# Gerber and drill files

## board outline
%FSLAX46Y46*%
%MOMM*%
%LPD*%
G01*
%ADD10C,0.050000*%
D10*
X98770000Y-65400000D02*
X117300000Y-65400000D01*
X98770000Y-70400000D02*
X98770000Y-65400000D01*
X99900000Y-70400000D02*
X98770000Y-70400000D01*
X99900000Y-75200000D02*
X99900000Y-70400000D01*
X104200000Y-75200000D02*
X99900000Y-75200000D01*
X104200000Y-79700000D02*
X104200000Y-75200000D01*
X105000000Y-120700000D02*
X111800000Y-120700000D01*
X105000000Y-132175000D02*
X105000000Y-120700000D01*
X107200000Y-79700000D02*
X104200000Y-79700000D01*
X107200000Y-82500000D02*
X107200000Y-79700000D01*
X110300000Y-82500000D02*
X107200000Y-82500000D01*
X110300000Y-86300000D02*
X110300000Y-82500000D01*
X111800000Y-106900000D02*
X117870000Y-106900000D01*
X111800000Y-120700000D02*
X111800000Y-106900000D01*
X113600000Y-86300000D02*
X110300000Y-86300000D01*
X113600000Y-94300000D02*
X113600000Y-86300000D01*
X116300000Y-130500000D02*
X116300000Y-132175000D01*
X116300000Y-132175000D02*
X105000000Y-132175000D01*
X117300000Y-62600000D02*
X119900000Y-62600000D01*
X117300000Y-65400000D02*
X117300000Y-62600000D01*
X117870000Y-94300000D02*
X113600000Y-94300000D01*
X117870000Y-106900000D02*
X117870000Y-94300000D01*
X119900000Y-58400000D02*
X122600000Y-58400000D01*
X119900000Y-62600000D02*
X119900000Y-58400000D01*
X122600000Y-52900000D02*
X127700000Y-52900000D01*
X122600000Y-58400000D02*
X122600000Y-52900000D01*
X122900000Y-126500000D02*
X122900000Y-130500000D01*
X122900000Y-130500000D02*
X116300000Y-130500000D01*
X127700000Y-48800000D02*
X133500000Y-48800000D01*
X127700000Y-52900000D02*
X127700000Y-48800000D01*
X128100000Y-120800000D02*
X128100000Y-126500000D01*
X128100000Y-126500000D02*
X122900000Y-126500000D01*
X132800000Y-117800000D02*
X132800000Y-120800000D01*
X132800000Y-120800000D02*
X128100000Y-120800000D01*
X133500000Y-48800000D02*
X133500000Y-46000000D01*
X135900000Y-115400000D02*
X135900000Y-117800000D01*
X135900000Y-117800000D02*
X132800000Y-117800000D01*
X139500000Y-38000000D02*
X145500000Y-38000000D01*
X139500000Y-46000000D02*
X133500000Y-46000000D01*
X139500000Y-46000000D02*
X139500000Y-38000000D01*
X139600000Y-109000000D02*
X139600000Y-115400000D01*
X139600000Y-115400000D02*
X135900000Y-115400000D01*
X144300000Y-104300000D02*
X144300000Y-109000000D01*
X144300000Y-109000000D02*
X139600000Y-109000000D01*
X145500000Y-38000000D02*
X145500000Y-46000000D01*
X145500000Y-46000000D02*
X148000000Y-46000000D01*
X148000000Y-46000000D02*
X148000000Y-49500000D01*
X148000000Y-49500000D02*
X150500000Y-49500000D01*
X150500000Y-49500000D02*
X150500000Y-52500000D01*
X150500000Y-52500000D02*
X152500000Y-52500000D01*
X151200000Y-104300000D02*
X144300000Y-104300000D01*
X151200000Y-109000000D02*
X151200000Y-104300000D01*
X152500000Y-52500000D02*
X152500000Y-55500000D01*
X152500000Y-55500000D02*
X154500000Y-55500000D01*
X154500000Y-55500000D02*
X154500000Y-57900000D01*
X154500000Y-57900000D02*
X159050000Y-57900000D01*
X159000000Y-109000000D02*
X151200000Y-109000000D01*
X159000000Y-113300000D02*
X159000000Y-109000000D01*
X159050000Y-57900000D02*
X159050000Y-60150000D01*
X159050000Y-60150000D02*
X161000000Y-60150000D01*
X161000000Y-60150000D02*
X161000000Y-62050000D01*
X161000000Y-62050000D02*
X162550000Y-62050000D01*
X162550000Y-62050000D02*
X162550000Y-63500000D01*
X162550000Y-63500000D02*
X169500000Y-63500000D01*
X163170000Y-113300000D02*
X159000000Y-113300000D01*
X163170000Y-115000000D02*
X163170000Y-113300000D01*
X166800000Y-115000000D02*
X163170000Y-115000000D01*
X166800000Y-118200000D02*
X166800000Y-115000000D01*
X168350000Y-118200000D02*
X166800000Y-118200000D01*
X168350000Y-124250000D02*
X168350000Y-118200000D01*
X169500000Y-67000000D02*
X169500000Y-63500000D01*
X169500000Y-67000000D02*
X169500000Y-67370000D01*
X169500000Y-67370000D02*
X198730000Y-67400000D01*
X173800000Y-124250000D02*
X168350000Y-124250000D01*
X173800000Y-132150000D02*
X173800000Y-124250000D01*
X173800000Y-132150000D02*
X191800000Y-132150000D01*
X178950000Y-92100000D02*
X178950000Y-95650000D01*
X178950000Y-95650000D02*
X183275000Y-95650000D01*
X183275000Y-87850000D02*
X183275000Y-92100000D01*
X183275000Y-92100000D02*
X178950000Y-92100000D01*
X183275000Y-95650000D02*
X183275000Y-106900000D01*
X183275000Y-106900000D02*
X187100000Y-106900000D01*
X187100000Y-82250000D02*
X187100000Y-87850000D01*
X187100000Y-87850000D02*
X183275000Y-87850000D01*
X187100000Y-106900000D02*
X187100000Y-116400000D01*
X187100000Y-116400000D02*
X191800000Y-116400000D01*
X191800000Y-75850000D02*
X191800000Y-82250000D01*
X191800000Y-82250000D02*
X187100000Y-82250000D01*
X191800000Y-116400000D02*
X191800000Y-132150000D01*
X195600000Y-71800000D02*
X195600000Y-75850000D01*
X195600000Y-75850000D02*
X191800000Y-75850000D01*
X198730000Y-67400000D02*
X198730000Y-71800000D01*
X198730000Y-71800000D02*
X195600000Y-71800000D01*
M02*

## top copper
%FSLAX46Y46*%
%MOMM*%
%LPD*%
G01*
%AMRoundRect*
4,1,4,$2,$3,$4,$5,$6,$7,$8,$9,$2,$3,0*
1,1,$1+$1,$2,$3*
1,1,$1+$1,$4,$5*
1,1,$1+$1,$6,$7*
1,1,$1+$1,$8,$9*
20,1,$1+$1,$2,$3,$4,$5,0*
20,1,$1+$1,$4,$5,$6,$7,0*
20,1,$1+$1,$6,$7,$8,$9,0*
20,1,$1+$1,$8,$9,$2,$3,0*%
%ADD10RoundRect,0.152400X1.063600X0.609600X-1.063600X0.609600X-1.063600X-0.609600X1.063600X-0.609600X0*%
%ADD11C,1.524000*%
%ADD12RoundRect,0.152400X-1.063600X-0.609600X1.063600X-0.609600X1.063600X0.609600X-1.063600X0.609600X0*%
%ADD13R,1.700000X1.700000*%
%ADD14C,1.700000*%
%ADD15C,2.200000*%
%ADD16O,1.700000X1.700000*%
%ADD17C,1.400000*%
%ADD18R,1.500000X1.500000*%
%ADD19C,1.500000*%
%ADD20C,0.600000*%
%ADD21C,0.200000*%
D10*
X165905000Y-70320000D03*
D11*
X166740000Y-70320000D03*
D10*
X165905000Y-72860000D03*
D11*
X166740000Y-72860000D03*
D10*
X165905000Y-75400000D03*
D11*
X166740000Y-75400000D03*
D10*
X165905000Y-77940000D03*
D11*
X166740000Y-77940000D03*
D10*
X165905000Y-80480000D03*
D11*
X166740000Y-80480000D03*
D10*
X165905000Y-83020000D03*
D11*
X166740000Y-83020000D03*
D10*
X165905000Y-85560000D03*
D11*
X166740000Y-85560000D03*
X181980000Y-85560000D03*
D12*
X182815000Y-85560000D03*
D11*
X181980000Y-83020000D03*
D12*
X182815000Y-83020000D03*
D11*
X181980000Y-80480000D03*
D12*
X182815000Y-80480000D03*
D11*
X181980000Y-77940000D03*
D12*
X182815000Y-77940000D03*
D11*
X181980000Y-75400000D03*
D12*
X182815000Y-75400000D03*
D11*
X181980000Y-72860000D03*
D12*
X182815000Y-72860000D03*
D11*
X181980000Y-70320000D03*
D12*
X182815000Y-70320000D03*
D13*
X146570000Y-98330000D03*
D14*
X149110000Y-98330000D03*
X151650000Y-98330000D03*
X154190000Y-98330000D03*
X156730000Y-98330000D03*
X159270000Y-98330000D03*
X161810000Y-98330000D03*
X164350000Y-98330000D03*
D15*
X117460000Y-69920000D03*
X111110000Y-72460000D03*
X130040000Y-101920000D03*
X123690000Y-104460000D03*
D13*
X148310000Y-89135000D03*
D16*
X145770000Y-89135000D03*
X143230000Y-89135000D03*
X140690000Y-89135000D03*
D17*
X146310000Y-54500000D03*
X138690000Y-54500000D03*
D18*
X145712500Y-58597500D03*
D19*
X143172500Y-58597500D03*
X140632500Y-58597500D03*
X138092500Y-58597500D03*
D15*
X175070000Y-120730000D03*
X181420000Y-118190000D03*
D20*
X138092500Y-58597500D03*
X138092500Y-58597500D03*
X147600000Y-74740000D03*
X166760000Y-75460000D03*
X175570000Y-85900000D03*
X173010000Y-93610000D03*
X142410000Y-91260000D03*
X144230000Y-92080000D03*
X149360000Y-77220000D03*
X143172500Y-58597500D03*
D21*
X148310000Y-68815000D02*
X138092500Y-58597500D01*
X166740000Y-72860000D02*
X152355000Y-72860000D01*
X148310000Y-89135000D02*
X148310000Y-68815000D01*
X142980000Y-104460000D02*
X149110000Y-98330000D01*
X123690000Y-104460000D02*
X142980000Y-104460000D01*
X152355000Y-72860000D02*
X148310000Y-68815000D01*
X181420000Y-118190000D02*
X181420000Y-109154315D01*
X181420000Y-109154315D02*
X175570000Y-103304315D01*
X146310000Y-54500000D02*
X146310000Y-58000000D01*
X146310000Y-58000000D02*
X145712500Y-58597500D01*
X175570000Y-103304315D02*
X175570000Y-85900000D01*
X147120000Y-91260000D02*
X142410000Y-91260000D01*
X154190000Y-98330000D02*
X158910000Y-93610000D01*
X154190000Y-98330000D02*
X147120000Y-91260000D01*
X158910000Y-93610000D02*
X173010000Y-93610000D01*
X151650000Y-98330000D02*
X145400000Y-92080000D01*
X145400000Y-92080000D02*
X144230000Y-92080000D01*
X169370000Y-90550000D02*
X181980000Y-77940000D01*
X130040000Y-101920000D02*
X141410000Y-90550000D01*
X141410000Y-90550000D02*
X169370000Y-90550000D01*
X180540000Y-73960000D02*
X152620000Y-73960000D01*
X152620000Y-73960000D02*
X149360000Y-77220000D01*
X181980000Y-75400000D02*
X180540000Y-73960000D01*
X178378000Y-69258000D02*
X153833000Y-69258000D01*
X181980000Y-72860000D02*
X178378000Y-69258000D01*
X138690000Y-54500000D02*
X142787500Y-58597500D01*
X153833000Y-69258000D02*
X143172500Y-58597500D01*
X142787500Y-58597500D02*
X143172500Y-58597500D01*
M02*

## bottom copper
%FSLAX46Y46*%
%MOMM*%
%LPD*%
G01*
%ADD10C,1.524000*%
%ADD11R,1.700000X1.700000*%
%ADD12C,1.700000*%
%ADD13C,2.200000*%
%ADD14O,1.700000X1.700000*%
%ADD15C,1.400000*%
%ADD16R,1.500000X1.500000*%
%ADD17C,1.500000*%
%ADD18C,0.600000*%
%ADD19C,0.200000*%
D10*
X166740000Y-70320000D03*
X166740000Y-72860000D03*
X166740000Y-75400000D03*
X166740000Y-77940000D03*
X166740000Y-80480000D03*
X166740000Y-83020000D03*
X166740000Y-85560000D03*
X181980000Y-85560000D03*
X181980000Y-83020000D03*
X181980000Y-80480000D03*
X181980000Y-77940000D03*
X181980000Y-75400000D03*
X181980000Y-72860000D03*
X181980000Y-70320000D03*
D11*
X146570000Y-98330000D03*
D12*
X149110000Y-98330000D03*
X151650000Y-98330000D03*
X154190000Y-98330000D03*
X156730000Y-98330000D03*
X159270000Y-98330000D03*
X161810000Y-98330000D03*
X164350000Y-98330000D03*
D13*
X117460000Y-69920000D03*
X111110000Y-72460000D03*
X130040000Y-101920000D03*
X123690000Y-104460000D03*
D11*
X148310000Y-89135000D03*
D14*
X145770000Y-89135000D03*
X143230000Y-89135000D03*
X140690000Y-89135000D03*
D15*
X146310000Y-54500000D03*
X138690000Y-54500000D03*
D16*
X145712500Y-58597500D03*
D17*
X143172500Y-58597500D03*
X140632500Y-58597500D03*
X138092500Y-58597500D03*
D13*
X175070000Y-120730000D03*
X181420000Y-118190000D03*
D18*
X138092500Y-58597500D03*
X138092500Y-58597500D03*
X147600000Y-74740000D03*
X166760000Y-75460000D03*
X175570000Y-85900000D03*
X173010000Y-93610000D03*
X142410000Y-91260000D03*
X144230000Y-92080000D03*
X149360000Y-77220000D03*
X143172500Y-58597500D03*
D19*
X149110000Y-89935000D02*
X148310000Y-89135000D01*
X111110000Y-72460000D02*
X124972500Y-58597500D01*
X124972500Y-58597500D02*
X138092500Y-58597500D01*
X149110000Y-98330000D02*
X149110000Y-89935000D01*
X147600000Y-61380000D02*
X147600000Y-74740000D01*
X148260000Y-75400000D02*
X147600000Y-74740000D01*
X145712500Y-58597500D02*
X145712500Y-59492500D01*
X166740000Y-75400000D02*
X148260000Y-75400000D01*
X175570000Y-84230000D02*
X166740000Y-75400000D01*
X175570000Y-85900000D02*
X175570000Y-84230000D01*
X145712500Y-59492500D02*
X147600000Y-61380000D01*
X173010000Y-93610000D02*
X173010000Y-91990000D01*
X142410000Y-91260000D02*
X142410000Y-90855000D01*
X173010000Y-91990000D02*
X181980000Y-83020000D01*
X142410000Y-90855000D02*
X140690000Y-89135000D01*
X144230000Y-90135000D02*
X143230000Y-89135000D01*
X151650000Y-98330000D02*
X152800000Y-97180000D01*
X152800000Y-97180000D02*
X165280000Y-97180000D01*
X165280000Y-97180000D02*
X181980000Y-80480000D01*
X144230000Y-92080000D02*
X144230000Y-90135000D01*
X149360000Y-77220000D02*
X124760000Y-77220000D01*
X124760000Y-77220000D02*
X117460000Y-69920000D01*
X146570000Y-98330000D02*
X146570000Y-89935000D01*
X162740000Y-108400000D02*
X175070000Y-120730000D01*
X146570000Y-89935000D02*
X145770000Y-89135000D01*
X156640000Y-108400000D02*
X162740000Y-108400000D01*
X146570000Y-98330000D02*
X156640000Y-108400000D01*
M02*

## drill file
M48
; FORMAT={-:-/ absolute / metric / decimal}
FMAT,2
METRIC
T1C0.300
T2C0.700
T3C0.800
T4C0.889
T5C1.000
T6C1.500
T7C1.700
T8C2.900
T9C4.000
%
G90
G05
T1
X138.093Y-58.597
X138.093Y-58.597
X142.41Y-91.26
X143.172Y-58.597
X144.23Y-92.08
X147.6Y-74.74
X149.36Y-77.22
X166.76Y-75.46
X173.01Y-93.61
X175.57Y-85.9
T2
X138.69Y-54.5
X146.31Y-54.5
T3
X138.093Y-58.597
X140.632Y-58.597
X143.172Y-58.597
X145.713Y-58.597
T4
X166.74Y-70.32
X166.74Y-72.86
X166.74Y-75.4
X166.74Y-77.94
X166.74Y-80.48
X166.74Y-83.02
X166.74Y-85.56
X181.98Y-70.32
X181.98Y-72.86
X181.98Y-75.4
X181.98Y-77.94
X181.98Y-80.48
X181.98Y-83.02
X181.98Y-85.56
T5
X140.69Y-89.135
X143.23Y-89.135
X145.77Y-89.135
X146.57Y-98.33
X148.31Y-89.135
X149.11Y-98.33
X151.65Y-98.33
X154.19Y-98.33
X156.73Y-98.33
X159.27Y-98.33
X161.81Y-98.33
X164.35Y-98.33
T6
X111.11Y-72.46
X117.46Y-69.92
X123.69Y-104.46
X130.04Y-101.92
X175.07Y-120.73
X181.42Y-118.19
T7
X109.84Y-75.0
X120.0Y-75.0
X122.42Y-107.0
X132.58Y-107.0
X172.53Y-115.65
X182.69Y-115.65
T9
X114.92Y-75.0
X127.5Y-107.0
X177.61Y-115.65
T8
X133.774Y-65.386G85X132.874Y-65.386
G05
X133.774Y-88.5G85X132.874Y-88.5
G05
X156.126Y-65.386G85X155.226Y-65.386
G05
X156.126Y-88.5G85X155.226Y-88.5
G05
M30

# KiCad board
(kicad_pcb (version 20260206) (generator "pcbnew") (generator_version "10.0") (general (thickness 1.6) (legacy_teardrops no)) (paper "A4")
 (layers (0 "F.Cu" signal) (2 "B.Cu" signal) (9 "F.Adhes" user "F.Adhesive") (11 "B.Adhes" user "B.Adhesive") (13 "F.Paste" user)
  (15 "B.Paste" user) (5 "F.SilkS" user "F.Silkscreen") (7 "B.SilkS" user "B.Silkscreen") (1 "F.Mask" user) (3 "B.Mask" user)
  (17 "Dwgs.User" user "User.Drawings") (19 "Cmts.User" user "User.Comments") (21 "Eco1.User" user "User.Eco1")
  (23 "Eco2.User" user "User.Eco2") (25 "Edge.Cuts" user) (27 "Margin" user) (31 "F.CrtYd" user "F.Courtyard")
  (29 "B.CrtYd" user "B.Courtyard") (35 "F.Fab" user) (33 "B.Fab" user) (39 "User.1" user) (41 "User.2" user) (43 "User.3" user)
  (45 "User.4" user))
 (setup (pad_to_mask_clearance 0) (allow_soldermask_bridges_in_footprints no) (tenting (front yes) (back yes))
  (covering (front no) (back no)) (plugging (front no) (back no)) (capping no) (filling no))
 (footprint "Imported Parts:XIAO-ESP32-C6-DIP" (layer "F.Cu") (at 174.36 77.94 90)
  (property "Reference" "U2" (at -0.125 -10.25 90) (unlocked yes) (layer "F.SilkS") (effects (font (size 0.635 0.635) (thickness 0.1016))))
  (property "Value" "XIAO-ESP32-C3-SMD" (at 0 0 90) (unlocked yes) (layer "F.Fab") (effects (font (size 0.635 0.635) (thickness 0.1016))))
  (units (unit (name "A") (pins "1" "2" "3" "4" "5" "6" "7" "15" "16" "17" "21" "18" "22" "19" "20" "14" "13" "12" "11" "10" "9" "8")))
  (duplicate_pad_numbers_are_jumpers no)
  (pad "1" smd roundrect (at 7.62 -8.455 180) (size 2.432 1.524) (layers "F.Cu" "F.Mask") (roundrect_rratio 0.1) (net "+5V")
   (thermal_bridge_angle 45))
  (pad "1" thru_hole circle (at 7.62 -7.62 180) (size 1.524 1.524) (drill 0.889) (layers "*.Cu" "*.Mask") (remove_unused_layers no)
   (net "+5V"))
  (pad "2" smd roundrect (at 5.08 -8.455 180) (size 2.432 1.524) (layers "F.Cu" "F.Mask") (roundrect_rratio 0.1) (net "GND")
   (thermal_bridge_angle 45))
  (pad "2" thru_hole circle (at 5.08 -7.62 180) (size 1.524 1.524) (drill 0.889) (layers "*.Cu" "*.Mask") (remove_unused_layers no)
   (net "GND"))
  (pad "3" smd roundrect (at 2.54 -8.455 180) (size 2.432 1.524) (layers "F.Cu" "F.Mask") (roundrect_rratio 0.1) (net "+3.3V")
   (thermal_bridge_angle 45))
  (pad "3" thru_hole circle (at 2.54 -7.62 180) (size 1.524 1.524) (drill 0.889) (layers "*.Cu" "*.Mask") (remove_unused_layers no)
   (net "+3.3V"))
  (pad "4" smd roundrect (at 0 -8.455 180) (size 2.432 1.524) (layers "F.Cu" "F.Mask") (roundrect_rratio 0.1)
   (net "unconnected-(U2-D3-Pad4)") (thermal_bridge_angle 45))
  (pad "4" thru_hole circle (at 0 -7.62 180) (size 1.524 1.524) (drill 0.889) (layers "*.Cu" "*.Mask") (remove_unused_layers no)
   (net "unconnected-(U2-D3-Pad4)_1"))
  (pad "5" smd roundrect (at -2.54 -8.455 180) (size 2.432 1.524) (layers "F.Cu" "F.Mask") (roundrect_rratio 0.1)
   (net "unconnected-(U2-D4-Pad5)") (thermal_bridge_angle 45))
  (pad "5" thru_hole circle (at -2.54 -7.62 180) (size 1.524 1.524) (drill 0.889) (layers "*.Cu" "*.Mask") (remove_unused_layers no)
   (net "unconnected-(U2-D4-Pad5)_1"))
  (pad "6" smd roundrect (at -5.08 -8.455 180) (size 2.432 1.524) (layers "F.Cu" "F.Mask") (roundrect_rratio 0.1)
   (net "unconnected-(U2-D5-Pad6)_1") (thermal_bridge_angle 45))
  (pad "6" thru_hole circle (at -5.08 -7.62 180) (size 1.524 1.524) (drill 0.889) (layers "*.Cu" "*.Mask") (remove_unused_layers no)
   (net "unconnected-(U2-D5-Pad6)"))
  (pad "7" smd roundrect (at -7.62 -8.455 180) (size 2.432 1.524) (layers "F.Cu" "F.Mask") (roundrect_rratio 0.1)
   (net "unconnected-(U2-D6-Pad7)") (thermal_bridge_angle 45))
  (pad "7" thru_hole circle (at -7.62 -7.62 180) (size 1.524 1.524) (drill 0.889) (layers "*.Cu" "*.Mask") (remove_unused_layers no)
   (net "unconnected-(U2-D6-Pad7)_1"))
  (pad "8" thru_hole circle (at -7.62 7.62) (size 1.524 1.524) (drill 0.889) (layers "*.Cu" "*.Mask") (remove_unused_layers no)
   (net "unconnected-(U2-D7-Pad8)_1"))
  (pad "8" smd roundrect (at -7.62 8.455) (size 2.432 1.524) (layers "F.Cu" "F.Mask") (roundrect_rratio 0.1)
   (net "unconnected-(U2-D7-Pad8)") (thermal_bridge_angle 45))
  (pad "9" thru_hole circle (at -5.08 7.62) (size 1.524 1.524) (drill 0.889) (layers "*.Cu" "*.Mask") (remove_unused_layers no) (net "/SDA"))
  (pad "9" smd roundrect (at -5.08 8.455) (size 2.432 1.524) (layers "F.Cu" "F.Mask") (roundrect_rratio 0.1) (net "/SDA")
   (thermal_bridge_angle 45))
  (pad "10" thru_hole circle (at -2.54 7.62) (size 1.524 1.524) (drill 0.889) (layers "*.Cu" "*.Mask") (remove_unused_layers no)
   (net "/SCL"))
  (pad "10" smd roundrect (at -2.54 8.455) (size 2.432 1.524) (layers "F.Cu" "F.Mask") (roundrect_rratio 0.1) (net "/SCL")
   (thermal_bridge_angle 45))
  (pad "11" thru_hole circle (at 0 7.62) (size 1.524 1.524) (drill 0.889) (layers "*.Cu" "*.Mask") (remove_unused_layers no) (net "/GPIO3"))
  (pad "11" smd roundrect (at 0 8.455) (size 2.432 1.524) (layers "F.Cu" "F.Mask") (roundrect_rratio 0.1) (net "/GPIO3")
   (thermal_bridge_angle 45))
  (pad "12" thru_hole circle (at 2.54 7.62) (size 1.524 1.524) (drill 0.889) (layers "*.Cu" "*.Mask") (remove_unused_layers no)
   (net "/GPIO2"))
  (pad "12" smd roundrect (at 2.54 8.455) (size 2.432 1.524) (layers "F.Cu" "F.Mask") (roundrect_rratio 0.1) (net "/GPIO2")
   (thermal_bridge_angle 45))
  (pad "13" thru_hole circle (at 5.08 7.62) (size 1.524 1.524) (drill 0.889) (layers "*.Cu" "*.Mask") (remove_unused_layers no)
   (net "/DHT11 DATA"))
  (pad "13" smd roundrect (at 5.08 8.455) (size 2.432 1.524) (layers "F.Cu" "F.Mask") (roundrect_rratio 0.1) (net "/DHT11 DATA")
   (thermal_bridge_angle 45))
  (pad "14" thru_hole circle (at 7.62 7.62) (size 1.524 1.524) (drill 0.889) (layers "*.Cu" "*.Mask") (remove_unused_layers no)
   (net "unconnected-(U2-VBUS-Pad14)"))
  (pad "14" smd roundrect (at 7.62 8.455) (size 2.432 1.524) (layers "F.Cu" "F.Mask") (roundrect_rratio 0.1)
   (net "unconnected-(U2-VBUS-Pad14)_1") (thermal_bridge_angle 45)))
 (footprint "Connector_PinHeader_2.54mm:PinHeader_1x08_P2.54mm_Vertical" (layer "F.Cu") (at 146.57 98.33 90)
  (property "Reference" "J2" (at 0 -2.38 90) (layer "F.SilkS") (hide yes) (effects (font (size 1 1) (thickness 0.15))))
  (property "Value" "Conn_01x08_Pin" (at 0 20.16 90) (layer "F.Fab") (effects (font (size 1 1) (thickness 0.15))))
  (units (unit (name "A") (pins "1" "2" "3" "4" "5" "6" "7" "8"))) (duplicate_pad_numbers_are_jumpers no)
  (pad "1" thru_hole rect (at 0 0 90) (size 1.7 1.7) (drill 1) (layers "*.Cu" "*.Mask") (remove_unused_layers no) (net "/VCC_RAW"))
  (pad "2" thru_hole circle (at 0 2.54 90) (size 1.7 1.7) (drill 1) (layers "*.Cu" "*.Mask") (remove_unused_layers no) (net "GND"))
  (pad "3" thru_hole circle (at 0 5.08 90) (size 1.7 1.7) (drill 1) (layers "*.Cu" "*.Mask") (remove_unused_layers no) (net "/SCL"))
  (pad "4" thru_hole circle (at 0 7.62 90) (size 1.7 1.7) (drill 1) (layers "*.Cu" "*.Mask") (remove_unused_layers no) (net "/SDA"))
  (pad "5" thru_hole circle (at 0 10.16 90) (size 1.7 1.7) (drill 1) (layers "*.Cu" "*.Mask") (remove_unused_layers no)
   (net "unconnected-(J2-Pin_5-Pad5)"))
  (pad "6" thru_hole circle (at 0 12.7 90) (size 1.7 1.7) (drill 1) (layers "*.Cu" "*.Mask") (remove_unused_layers no)
   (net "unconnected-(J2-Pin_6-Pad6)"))
  (pad "7" thru_hole circle (at 0 15.24 90) (size 1.7 1.7) (drill 1) (layers "*.Cu" "*.Mask") (remove_unused_layers no)
   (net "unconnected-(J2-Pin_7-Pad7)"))
  (pad "8" thru_hole circle (at 0 17.78 90) (size 1.7 1.7) (drill 1) (layers "*.Cu" "*.Mask") (remove_unused_layers no)
   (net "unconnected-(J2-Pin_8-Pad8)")))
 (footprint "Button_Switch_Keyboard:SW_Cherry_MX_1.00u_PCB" (layer "F.Cu") (at 117.46 69.92)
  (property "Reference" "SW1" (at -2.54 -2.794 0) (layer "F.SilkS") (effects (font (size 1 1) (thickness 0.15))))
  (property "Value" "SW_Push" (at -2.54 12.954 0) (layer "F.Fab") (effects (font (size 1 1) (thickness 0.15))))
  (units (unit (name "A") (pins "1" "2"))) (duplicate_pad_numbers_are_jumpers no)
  (pad "" np_thru_hole circle (at -7.62 5.08) (size 1.7 1.7) (drill 1.7) (layers "*.Cu" "*.Mask"))
  (pad "" np_thru_hole circle (at -2.54 5.08) (size 4 4) (drill 4) (layers "*.Cu" "*.Mask"))
  (pad "" np_thru_hole circle (at 2.54 5.08) (size 1.7 1.7) (drill 1.7) (layers "*.Cu" "*.Mask"))
  (pad "1" thru_hole circle (at 0 0) (size 2.2 2.2) (drill 1.5) (layers "*.Cu" "*.Mask") (remove_unused_layers no) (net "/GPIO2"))
  (pad "2" thru_hole circle (at -6.35 2.54) (size 2.2 2.2) (drill 1.5) (layers "*.Cu" "*.Mask") (remove_unused_layers no) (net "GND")))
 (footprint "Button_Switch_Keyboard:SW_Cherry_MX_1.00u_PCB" (layer "F.Cu") (at 130.04 101.92)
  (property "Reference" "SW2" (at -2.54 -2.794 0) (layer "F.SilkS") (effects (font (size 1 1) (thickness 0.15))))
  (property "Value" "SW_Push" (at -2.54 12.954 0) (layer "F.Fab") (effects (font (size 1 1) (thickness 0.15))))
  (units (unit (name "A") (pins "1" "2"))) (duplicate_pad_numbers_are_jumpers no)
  (pad "" np_thru_hole circle (at -7.62 5.08) (size 1.7 1.7) (drill 1.7) (layers "*.Cu" "*.Mask"))
  (pad "" np_thru_hole circle (at -2.54 5.08) (size 4 4) (drill 4) (layers "*.Cu" "*.Mask"))
  (pad "" np_thru_hole circle (at 2.54 5.08) (size 1.7 1.7) (drill 1.7) (layers "*.Cu" "*.Mask"))
  (pad "1" thru_hole circle (at 0 0) (size 2.2 2.2) (drill 1.5) (layers "*.Cu" "*.Mask") (remove_unused_layers no) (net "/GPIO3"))
  (pad "2" thru_hole circle (at -6.35 2.54) (size 2.2 2.2) (drill 1.5) (layers "*.Cu" "*.Mask") (remove_unused_layers no) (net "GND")))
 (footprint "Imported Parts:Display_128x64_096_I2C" (layer "F.Cu") (at 144.5 89.135 180)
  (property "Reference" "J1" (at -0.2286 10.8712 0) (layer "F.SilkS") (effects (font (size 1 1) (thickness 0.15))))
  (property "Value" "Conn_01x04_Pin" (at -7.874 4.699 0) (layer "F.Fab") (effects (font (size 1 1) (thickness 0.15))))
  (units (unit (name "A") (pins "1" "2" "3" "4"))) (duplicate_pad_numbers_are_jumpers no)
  (pad "" np_thru_hole oval (at -11.176 0.635 180) (size 3.8 2.9) (drill oval 3.8 2.9) (layers "*.Cu" "*.Mask"))
  (pad "" np_thru_hole oval (at -11.176 23.749 180) (size 3.8 2.9) (drill oval 3.8 2.9) (layers "*.Cu" "*.Mask"))
  (pad "" np_thru_hole oval (at 11.176 0.635 180) (size 3.8 2.9) (drill oval 3.8 2.9) (layers "*.Cu" "*.Mask"))
  (pad "" np_thru_hole oval (at 11.176 23.749 180) (size 3.8 2.9) (drill oval 3.8 2.9) (layers "*.Cu" "*.Mask"))
  (pad "1" thru_hole rect (at -3.81 0 270) (size 1.7 1.7) (drill 1) (layers "*.Cu" "*.Mask") (remove_unused_layers no) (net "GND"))
  (pad "2" thru_hole oval (at -1.27 0 270) (size 1.7 1.7) (drill 1) (layers "*.Cu" "*.Mask") (remove_unused_layers no) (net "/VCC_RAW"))
  (pad "3" thru_hole oval (at 1.27 0 270) (size 1.7 1.7) (drill 1) (layers "*.Cu" "*.Mask") (remove_unused_layers no) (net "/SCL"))
  (pad "4" thru_hole oval (at 3.81 0 270) (size 1.7 1.7) (drill 1) (layers "*.Cu" "*.Mask") (remove_unused_layers no) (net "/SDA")))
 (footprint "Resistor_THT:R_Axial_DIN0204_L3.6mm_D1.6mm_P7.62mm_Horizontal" (layer "F.Cu") (at 146.31 54.5 180)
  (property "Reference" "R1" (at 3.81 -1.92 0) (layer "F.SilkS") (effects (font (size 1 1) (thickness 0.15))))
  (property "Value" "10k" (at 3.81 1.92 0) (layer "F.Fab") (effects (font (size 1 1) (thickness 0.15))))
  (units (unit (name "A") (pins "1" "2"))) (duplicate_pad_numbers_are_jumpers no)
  (pad "1" thru_hole circle (at 0 0 180) (size 1.4 1.4) (drill 0.7) (layers "*.Cu" "*.Mask") (remove_unused_layers no) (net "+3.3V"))
  (pad "2" thru_hole circle (at 7.62 0 180) (size 1.4 1.4) (drill 0.7) (layers "*.Cu" "*.Mask") (remove_unused_layers no)
   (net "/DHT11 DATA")))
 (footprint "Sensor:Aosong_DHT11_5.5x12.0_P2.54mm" (layer "F.Cu") (at 145.7125 58.5975 -90)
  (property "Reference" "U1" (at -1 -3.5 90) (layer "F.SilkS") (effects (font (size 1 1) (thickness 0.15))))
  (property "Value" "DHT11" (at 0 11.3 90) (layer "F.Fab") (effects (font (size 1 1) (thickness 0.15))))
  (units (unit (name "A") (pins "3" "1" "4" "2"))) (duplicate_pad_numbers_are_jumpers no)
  (pad "1" thru_hole rect (at 0 0 270) (size 1.5 1.5) (drill 0.8) (layers "*.Cu" "*.Mask") (remove_unused_layers no) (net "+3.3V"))
  (pad "2" thru_hole circle (at 0 2.54 270) (size 1.5 1.5) (drill 0.8) (layers "*.Cu" "*.Mask") (remove_unused_layers no)
   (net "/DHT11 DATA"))
  (pad "3" thru_hole circle (at 0 5.08 270) (size 1.5 1.5) (drill 0.8) (layers "*.Cu" "*.Mask") (remove_unused_layers no)
   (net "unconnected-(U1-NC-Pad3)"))
  (pad "4" thru_hole circle (at 0 7.62 270) (size 1.5 1.5) (drill 0.8) (layers "*.Cu" "*.Mask") (remove_unused_layers no) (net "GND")))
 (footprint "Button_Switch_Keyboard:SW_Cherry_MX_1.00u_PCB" (layer "F.Cu") (at 175.07 120.73 180)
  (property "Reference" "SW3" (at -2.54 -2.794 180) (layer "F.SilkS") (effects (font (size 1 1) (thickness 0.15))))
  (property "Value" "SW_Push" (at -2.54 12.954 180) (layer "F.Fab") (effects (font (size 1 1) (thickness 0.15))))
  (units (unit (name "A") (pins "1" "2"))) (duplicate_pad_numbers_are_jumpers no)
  (pad "" np_thru_hole circle (at -7.62 5.08 180) (size 1.7 1.7) (drill 1.7) (layers "*.Cu" "*.Mask"))
  (pad "" np_thru_hole circle (at -2.54 5.08 180) (size 4 4) (drill 4) (layers "*.Cu" "*.Mask"))
  (pad "" np_thru_hole circle (at 2.54 5.08 180) (size 1.7 1.7) (drill 1.7) (layers "*.Cu" "*.Mask"))
  (pad "1" thru_hole circle (at 0 0 180) (size 2.2 2.2) (drill 1.5) (layers "*.Cu" "*.Mask") (remove_unused_layers no) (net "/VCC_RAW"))
  (pad "2" thru_hole circle (at -6.35 2.54 180) (size 2.2 2.2) (drill 1.5) (layers "*.Cu" "*.Mask") (remove_unused_layers no) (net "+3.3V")))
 (gr_line (start 98.77 65.4) (end 117.3 65.4) (stroke (width 0.05) (type default)) (layer "Edge.Cuts"))
 (gr_line (start 98.77 70.4) (end 98.77 65.4) (stroke (width 0.05) (type default)) (layer "Edge.Cuts"))
 (gr_line (start 99.9 70.4) (end 98.77 70.4) (stroke (width 0.05) (type default)) (layer "Edge.Cuts"))
 (gr_line (start 99.9 75.2) (end 99.9 70.4) (stroke (width 0.05) (type default)) (layer "Edge.Cuts"))
 (gr_line (start 104.2 75.2) (end 99.9 75.2) (stroke (width 0.05) (type default)) (layer "Edge.Cuts"))
 (gr_line (start 104.2 79.7) (end 104.2 75.2) (stroke (width 0.05) (type default)) (layer "Edge.Cuts"))
 (gr_line (start 105 120.7) (end 111.8 120.7) (stroke (width 0.05) (type default)) (layer "Edge.Cuts"))
 (gr_line (start 105 132.175) (end 105 120.7) (stroke (width 0.05) (type default)) (layer "Edge.Cuts"))
 (gr_line (start 107.2 79.7) (end 104.2 79.7) (stroke (width 0.05) (type default)) (layer "Edge.Cuts"))
 (gr_line (start 107.2 82.5) (end 107.2 79.7) (stroke (width 0.05) (type default)) (layer "Edge.Cuts"))
 (gr_line (start 110.3 82.5) (end 107.2 82.5) (stroke (width 0.05) (type default)) (layer "Edge.Cuts"))
 (gr_line (start 110.3 86.3) (end 110.3 82.5) (stroke (width 0.05) (type default)) (layer "Edge.Cuts"))
 (gr_line (start 111.8 106.9) (end 117.87 106.9) (stroke (width 0.05) (type default)) (layer "Edge.Cuts"))
 (gr_line (start 111.8 120.7) (end 111.8 106.9) (stroke (width 0.05) (type default)) (layer "Edge.Cuts"))
 (gr_line (start 113.6 86.3) (end 110.3 86.3) (stroke (width 0.05) (type default)) (layer "Edge.Cuts"))
 (gr_line (start 113.6 94.3) (end 113.6 86.3) (stroke (width 0.05) (type default)) (layer "Edge.Cuts"))
 (gr_line (start 116.3 130.5) (end 116.3 132.175) (stroke (width 0.05) (type default)) (layer "Edge.Cuts"))
 (gr_line (start 116.3 132.175) (end 105 132.175) (stroke (width 0.05) (type default)) (layer "Edge.Cuts"))
 (gr_line (start 117.3 62.6) (end 119.9 62.6) (stroke (width 0.05) (type default)) (layer "Edge.Cuts"))
 (gr_line (start 117.3 65.4) (end 117.3 62.6) (stroke (width 0.05) (type default)) (layer "Edge.Cuts"))
 (gr_line (start 117.87 94.3) (end 113.6 94.3) (stroke (width 0.05) (type default)) (layer "Edge.Cuts"))
 (gr_line (start 117.87 106.9) (end 117.87 94.3) (stroke (width 0.05) (type default)) (layer "Edge.Cuts"))
 (gr_line (start 119.9 58.4) (end 122.6 58.4) (stroke (width 0.05) (type default)) (layer "Edge.Cuts"))
 (gr_line (start 119.9 62.6) (end 119.9 58.4) (stroke (width 0.05) (type default)) (layer "Edge.Cuts"))
 (gr_line (start 122.6 52.9) (end 127.7 52.9) (stroke (width 0.05) (type default)) (layer "Edge.Cuts"))
 (gr_line (start 122.6 58.4) (end 122.6 52.9) (stroke (width 0.05) (type default)) (layer "Edge.Cuts"))
 (gr_line (start 122.9 126.5) (end 122.9 130.5) (stroke (width 0.05) (type default)) (layer "Edge.Cuts"))
 (gr_line (start 122.9 130.5) (end 116.3 130.5) (stroke (width 0.05) (type default)) (layer "Edge.Cuts"))
 (gr_line (start 127.7 48.8) (end 133.5 48.8) (stroke (width 0.05) (type default)) (layer "Edge.Cuts"))
 (gr_line (start 127.7 52.9) (end 127.7 48.8) (stroke (width 0.05) (type default)) (layer "Edge.Cuts"))
 (gr_line (start 128.1 120.8) (end 128.1 126.5) (stroke (width 0.05) (type default)) (layer "Edge.Cuts"))
 (gr_line (start 128.1 126.5) (end 122.9 126.5) (stroke (width 0.05) (type default)) (layer "Edge.Cuts"))
 (gr_line (start 132.8 117.8) (end 132.8 120.8) (stroke (width 0.05) (type default)) (layer "Edge.Cuts"))
 (gr_line (start 132.8 120.8) (end 128.1 120.8) (stroke (width 0.05) (type default)) (layer "Edge.Cuts"))
 (gr_line (start 133.5 48.8) (end 133.5 46) (stroke (width 0.05) (type default)) (layer "Edge.Cuts"))
 (gr_line (start 135.9 115.4) (end 135.9 117.8) (stroke (width 0.05) (type default)) (layer "Edge.Cuts"))
 (gr_line (start 135.9 117.8) (end 132.8 117.8) (stroke (width 0.05) (type default)) (layer "Edge.Cuts"))
 (gr_line (start 139.5 38) (end 145.5 38) (stroke (width 0.05) (type default)) (layer "Edge.Cuts"))
 (gr_line (start 139.5 46) (end 133.5 46) (stroke (width 0.05) (type default)) (layer "Edge.Cuts"))
 (gr_line (start 139.5 46) (end 139.5 38) (stroke (width 0.05) (type default)) (layer "Edge.Cuts"))
 (gr_line (start 139.6 109) (end 139.6 115.4) (stroke (width 0.05) (type default)) (layer "Edge.Cuts"))
 (gr_line (start 139.6 115.4) (end 135.9 115.4) (stroke (width 0.05) (type default)) (layer "Edge.Cuts"))
 (gr_line (start 144.3 104.3) (end 144.3 109) (stroke (width 0.05) (type default)) (layer "Edge.Cuts"))
 (gr_line (start 144.3 109) (end 139.6 109) (stroke (width 0.05) (type default)) (layer "Edge.Cuts"))
 (gr_line (start 145.5 38) (end 145.5 46) (stroke (width 0.05) (type default)) (layer "Edge.Cuts"))
 (gr_line (start 145.5 46) (end 148 46) (stroke (width 0.05) (type default)) (layer "Edge.Cuts"))
 (gr_line (start 148 46) (end 148 49.5) (stroke (width 0.05) (type default)) (layer "Edge.Cuts"))
 (gr_line (start 148 49.5) (end 150.5 49.5) (stroke (width 0.05) (type default)) (layer "Edge.Cuts"))
 (gr_line (start 150.5 49.5) (end 150.5 52.5) (stroke (width 0.05) (type default)) (layer "Edge.Cuts"))
 (gr_line (start 150.5 52.5) (end 152.5 52.5) (stroke (width 0.05) (type default)) (layer "Edge.Cuts"))
 (gr_line (start 151.2 104.3) (end 144.3 104.3) (stroke (width 0.05) (type default)) (layer "Edge.Cuts"))
 (gr_line (start 151.2 109) (end 151.2 104.3) (stroke (width 0.05) (type default)) (layer "Edge.Cuts"))
 (gr_line (start 152.5 52.5) (end 152.5 55.5) (stroke (width 0.05) (type default)) (layer "Edge.Cuts"))
 (gr_line (start 152.5 55.5) (end 154.5 55.5) (stroke (width 0.05) (type default)) (layer "Edge.Cuts"))
 (gr_line (start 154.5 55.5) (end 154.5 57.9) (stroke (width 0.05) (type default)) (layer "Edge.Cuts"))
 (gr_line (start 154.5 57.9) (end 159.05 57.9) (stroke (width 0.05) (type default)) (layer "Edge.Cuts"))
 (gr_line (start 159 109) (end 151.2 109) (stroke (width 0.05) (type default)) (layer "Edge.Cuts"))
 (gr_line (start 159 113.3) (end 159 109) (stroke (width 0.05) (type default)) (layer "Edge.Cuts"))
 (gr_line (start 159.05 57.9) (end 159.05 60.15) (stroke (width 0.05) (type solid)) (layer "Edge.Cuts"))
 (gr_line (start 159.05 60.15) (end 161 60.15) (stroke (width 0.05) (type default)) (layer "Edge.Cuts"))
 (gr_line (start 161 60.15) (end 161 62.05) (stroke (width 0.05) (type default)) (layer "Edge.Cuts"))
 (gr_line (start 161 62.05) (end 162.55 62.05) (stroke (width 0.05) (type default)) (layer "Edge.Cuts"))
 (gr_line (start 162.55 62.05) (end 162.55 63.5) (stroke (width 0.05) (type solid)) (layer "Edge.Cuts"))
 (gr_line (start 162.55 63.5) (end 169.5 63.5) (stroke (width 0.05) (type default)) (layer "Edge.Cuts"))
 (gr_line (start 163.17 113.3) (end 159 113.3) (stroke (width 0.05) (type default)) (layer "Edge.Cuts"))
 (gr_line (start 163.17 115) (end 163.17 113.3) (stroke (width 0.05) (type default)) (layer "Edge.Cuts"))
 (gr_line (start 166.8 115) (end 163.17 115) (stroke (width 0.05) (type default)) (layer "Edge.Cuts"))
 (gr_line (start 166.8 118.2) (end 166.8 115) (stroke (width 0.05) (type solid)) (layer "Edge.Cuts"))
 (gr_line (start 168.35 118.2) (end 166.8 118.2) (stroke (width 0.05) (type solid)) (layer "Edge.Cuts"))
 (gr_line (start 168.35 124.25) (end 168.35 118.2) (stroke (width 0.05) (type default)) (layer "Edge.Cuts"))
 (gr_line (start 169.5 67) (end 169.5 63.5) (stroke (width 0.05) (type default)) (layer "Edge.Cuts"))
 (gr_line (start 169.5 67) (end 169.5 67.37) (stroke (width 0.05) (type default)) (layer "Edge.Cuts"))
 (gr_line (start 169.5 67.37) (end 198.73 67.4) (stroke (width 0.05) (type default)) (layer "Edge.Cuts"))
 (gr_line (start 173.8 124.25) (end 168.35 124.25) (stroke (width 0.05) (type default)) (layer "Edge.Cuts"))
 (gr_line (start 173.8 132.15) (end 173.8 124.25) (stroke (width 0.05) (type default)) (layer "Edge.Cuts"))
 (gr_line (start 173.8 132.15) (end 191.8 132.15) (stroke (width 0.05) (type default)) (layer "Edge.Cuts"))
 (gr_line (start 178.95 92.1) (end 178.95 95.65) (stroke (width 0.05) (type default)) (layer "Edge.Cuts"))
 (gr_line (start 178.95 95.65) (end 183.275 95.65) (stroke (width 0.05) (type default)) (layer "Edge.Cuts"))
 (gr_line (start 183.275 87.85) (end 183.275 92.1) (stroke (width 0.05) (type default)) (layer "Edge.Cuts"))
 (gr_line (start 183.275 92.1) (end 178.95 92.1) (stroke (width 0.05) (type default)) (layer "Edge.Cuts"))
 (gr_line (start 183.275 95.65) (end 183.275 106.9) (stroke (width 0.05) (type default)) (layer "Edge.Cuts"))
 (gr_line (start 183.275 106.9) (end 187.1 106.9) (stroke (width 0.05) (type default)) (layer "Edge.Cuts"))
 (gr_line (start 187.1 82.25) (end 187.1 87.85) (stroke (width 0.05) (type default)) (layer "Edge.Cuts"))
 (gr_line (start 187.1 87.85) (end 183.275 87.85) (stroke (width 0.05) (type solid)) (layer "Edge.Cuts"))
 (gr_line (start 187.1 106.9) (end 187.1 116.4) (stroke (width 0.05) (type default)) (layer "Edge.Cuts"))
 (gr_line (start 187.1 116.4) (end 191.8 116.4) (stroke (width 0.05) (type default)) (layer "Edge.Cuts"))
 (gr_line (start 191.8 75.85) (end 191.8 82.25) (stroke (width 0.05) (type default)) (layer "Edge.Cuts"))
 (gr_line (start 191.8 82.25) (end 187.1 82.25) (stroke (width 0.05) (type default)) (layer "Edge.Cuts"))
 (gr_line (start 191.8 116.4) (end 191.8 132.15) (stroke (width 0.05) (type default)) (layer "Edge.Cuts"))
 (gr_line (start 195.6 71.8) (end 195.6 75.85) (stroke (width 0.05) (type default)) (layer "Edge.Cuts"))
 (gr_line (start 195.6 75.85) (end 191.8 75.85) (stroke (width 0.05) (type default)) (layer "Edge.Cuts"))
 (gr_line (start 198.73 67.4) (end 198.73 71.8) (stroke (width 0.05) (type default)) (layer "Edge.Cuts"))
 (gr_line (start 198.73 71.8) (end 195.6 71.8) (stroke (width 0.05) (type default)) (layer "Edge.Cuts"))
 (segment (start 148.31 68.815) (end 138.0925 58.5975) (width 0.2) (layer "F.Cu") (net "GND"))
 (segment (start 166.74 72.86) (end 152.355 72.86) (width 0.2) (layer "F.Cu") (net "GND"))
 (segment (start 148.31 89.135) (end 148.31 68.815) (width 0.2) (layer "F.Cu") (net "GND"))
 (segment (start 142.98 104.46) (end 149.11 98.33) (width 0.2) (layer "F.Cu") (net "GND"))
 (segment (start 123.69 104.46) (end 142.98 104.46) (width 0.2) (layer "F.Cu") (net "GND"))
 (segment (start 152.355 72.86) (end 148.31 68.815) (width 0.2) (layer "F.Cu") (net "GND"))
 (via (at 138.0925 58.5975) (size 0.6) (drill 0.3) (layers "F.Cu" "B.Cu") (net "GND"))
 (via (at 138.0925 58.5975) (size 0.6) (drill 0.3) (layers "F.Cu" "B.Cu") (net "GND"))
 (segment (start 149.11 89.935) (end 148.31 89.135) (width 0.2) (layer "B.Cu") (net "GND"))
 (segment (start 111.11 72.46) (end 124.9725 58.5975) (width 0.2) (layer "B.Cu") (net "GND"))
 (segment (start 124.9725 58.5975) (end 138.0925 58.5975) (width 0.2) (layer "B.Cu") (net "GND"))
 (segment (start 149.11 98.33) (end 149.11 89.935) (width 0.2) (layer "B.Cu") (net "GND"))
 (segment (start 181.42 118.19) (end 181.42 109.154315) (width 0.2) (layer "F.Cu") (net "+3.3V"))
 (segment (start 181.42 109.154315) (end 175.57 103.304315) (width 0.2) (layer "F.Cu") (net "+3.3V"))
 (segment (start 146.31 54.5) (end 146.31 58) (width 0.2) (layer "F.Cu") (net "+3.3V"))
 (segment (start 146.31 58) (end 145.7125 58.5975) (width 0.2) (layer "F.Cu") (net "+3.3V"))
 (segment (start 175.57 103.304315) (end 175.57 85.9) (width 0.2) (layer "F.Cu") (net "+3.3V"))
 (via (at 147.6 74.74) (size 0.6) (drill 0.3) (layers "F.Cu" "B.Cu") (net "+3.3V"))
 (via (at 166.76 75.46) (size 0.6) (drill 0.3) (layers "F.Cu" "B.Cu") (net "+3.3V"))
 (via (at 175.57 85.9) (size 0.6) (drill 0.3) (layers "F.Cu" "B.Cu") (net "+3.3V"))
 (segment (start 147.6 61.38) (end 147.6 74.74) (width 0.2) (layer "B.Cu") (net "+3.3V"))
 (segment (start 148.26 75.4) (end 147.6 74.74) (width 0.2) (layer "B.Cu") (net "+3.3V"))
 (segment (start 145.7125 58.5975) (end 145.7125 59.4925) (width 0.2) (layer "B.Cu") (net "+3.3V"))
 (segment (start 166.74 75.4) (end 148.26 75.4) (width 0.2) (layer "B.Cu") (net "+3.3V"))
 (segment (start 175.57 84.23) (end 166.74 75.4) (width 0.2) (layer "B.Cu") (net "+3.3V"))
 (segment (start 175.57 85.9) (end 175.57 84.23) (width 0.2) (layer "B.Cu") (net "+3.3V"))
 (segment (start 145.7125 59.4925) (end 147.6 61.38) (width 0.2) (layer "B.Cu") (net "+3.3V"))
 (segment (start 147.12 91.26) (end 142.41 91.26) (width 0.2) (layer "F.Cu") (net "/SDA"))
 (segment (start 154.19 98.33) (end 158.91 93.61) (width 0.2) (layer "F.Cu") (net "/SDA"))
 (segment (start 154.19 98.33) (end 147.12 91.26) (width 0.2) (layer "F.Cu") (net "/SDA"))
 (segment (start 158.91 93.61) (end 173.01 93.61) (width 0.2) (layer "F.Cu") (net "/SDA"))
 (via (at 173.01 93.61) (size 0.6) (drill 0.3) (layers "F.Cu" "B.Cu") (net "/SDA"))
 (via (at 142.41 91.26) (size 0.6) (drill 0.3) (layers "F.Cu" "B.Cu") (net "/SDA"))
 (segment (start 173.01 93.61) (end 173.01 91.99) (width 0.2) (layer "B.Cu") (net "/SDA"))
 (segment (start 142.41 91.26) (end 142.41 90.855) (width 0.2) (layer "B.Cu") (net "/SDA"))
 (segment (start 173.01 91.99) (end 181.98 83.02) (width 0.2) (layer "B.Cu") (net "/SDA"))
 (segment (start 142.41 90.855) (end 140.69 89.135) (width 0.2) (layer "B.Cu") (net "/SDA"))
 (segment (start 151.65 98.33) (end 145.4 92.08) (width 0.2) (layer "F.Cu") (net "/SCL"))
 (segment (start 145.4 92.08) (end 144.23 92.08) (width 0.2) (layer "F.Cu") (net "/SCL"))
 (via (at 144.23 92.08) (size 0.6) (drill 0.3) (layers "F.Cu" "B.Cu") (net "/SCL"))
 (segment (start 144.23 90.135) (end 143.23 89.135) (width 0.2) (layer "B.Cu") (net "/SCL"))
 (segment (start 151.65 98.33) (end 152.8 97.18) (width 0.2) (layer "B.Cu") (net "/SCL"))
 (segment (start 152.8 97.18) (end 165.28 97.18) (width 0.2) (layer "B.Cu") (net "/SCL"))
 (segment (start 165.28 97.18) (end 181.98 80.48) (width 0.2) (layer "B.Cu") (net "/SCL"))
 (segment (start 144.23 92.08) (end 144.23 90.135) (width 0.2) (layer "B.Cu") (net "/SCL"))
 (segment (start 169.37 90.55) (end 181.98 77.94) (width 0.2) (layer "F.Cu") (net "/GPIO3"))
 (segment (start 130.04 101.92) (end 141.41 90.55) (width 0.2) (layer "F.Cu") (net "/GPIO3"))
 (segment (start 141.41 90.55) (end 169.37 90.55) (width 0.2) (layer "F.Cu") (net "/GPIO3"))
 (segment (start 180.54 73.96) (end 152.62 73.96) (width 0.2) (layer "F.Cu") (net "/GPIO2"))
 (segment (start 152.62 73.96) (end 149.36 77.22) (width 0.2) (layer "F.Cu") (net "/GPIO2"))
 (segment (start 181.98 75.4) (end 180.54 73.96) (width 0.2) (layer "F.Cu") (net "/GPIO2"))
 (via (at 149.36 77.22) (size 0.6) (drill 0.3) (layers "F.Cu" "B.Cu") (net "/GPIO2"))
 (segment (start 149.36 77.22) (end 124.76 77.22) (width 0.2) (layer "B.Cu") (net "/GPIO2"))
 (segment (start 124.76 77.22) (end 117.46 69.92) (width 0.2) (layer "B.Cu") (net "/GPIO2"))
 (segment (start 178.378 69.258) (end 153.833 69.258) (width 0.2) (layer "F.Cu") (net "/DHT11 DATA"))
 (segment (start 181.98 72.86) (end 178.378 69.258) (width 0.2) (layer "F.Cu") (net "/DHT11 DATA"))
 (segment (start 138.69 54.5) (end 142.7875 58.5975) (width 0.2) (layer "F.Cu") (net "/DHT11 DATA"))
 (segment (start 153.833 69.258) (end 143.1725 58.5975) (width 0.2) (layer "F.Cu") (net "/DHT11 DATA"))
 (segment (start 142.7875 58.5975) (end 143.1725 58.5975) (width 0.2) (layer "F.Cu") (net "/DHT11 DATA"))
 (via (at 143.1725 58.5975) (size 0.6) (drill 0.3) (layers "F.Cu" "B.Cu") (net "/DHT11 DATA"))
 (segment (start 146.57 98.33) (end 146.57 89.935) (width 0.2) (layer "B.Cu") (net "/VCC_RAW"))
 (segment (start 162.74 108.4) (end 175.07 120.73) (width 0.2) (layer "B.Cu") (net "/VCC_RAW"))
 (segment (start 146.57 89.935) (end 145.77 89.135) (width 0.2) (layer "B.Cu") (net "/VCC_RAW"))
 (segment (start 156.64 108.4) (end 162.74 108.4) (width 0.2) (layer "B.Cu") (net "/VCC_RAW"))
 (segment (start 146.57 98.33) (end 156.64 108.4) (width 0.2) (layer "B.Cu") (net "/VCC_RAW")))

